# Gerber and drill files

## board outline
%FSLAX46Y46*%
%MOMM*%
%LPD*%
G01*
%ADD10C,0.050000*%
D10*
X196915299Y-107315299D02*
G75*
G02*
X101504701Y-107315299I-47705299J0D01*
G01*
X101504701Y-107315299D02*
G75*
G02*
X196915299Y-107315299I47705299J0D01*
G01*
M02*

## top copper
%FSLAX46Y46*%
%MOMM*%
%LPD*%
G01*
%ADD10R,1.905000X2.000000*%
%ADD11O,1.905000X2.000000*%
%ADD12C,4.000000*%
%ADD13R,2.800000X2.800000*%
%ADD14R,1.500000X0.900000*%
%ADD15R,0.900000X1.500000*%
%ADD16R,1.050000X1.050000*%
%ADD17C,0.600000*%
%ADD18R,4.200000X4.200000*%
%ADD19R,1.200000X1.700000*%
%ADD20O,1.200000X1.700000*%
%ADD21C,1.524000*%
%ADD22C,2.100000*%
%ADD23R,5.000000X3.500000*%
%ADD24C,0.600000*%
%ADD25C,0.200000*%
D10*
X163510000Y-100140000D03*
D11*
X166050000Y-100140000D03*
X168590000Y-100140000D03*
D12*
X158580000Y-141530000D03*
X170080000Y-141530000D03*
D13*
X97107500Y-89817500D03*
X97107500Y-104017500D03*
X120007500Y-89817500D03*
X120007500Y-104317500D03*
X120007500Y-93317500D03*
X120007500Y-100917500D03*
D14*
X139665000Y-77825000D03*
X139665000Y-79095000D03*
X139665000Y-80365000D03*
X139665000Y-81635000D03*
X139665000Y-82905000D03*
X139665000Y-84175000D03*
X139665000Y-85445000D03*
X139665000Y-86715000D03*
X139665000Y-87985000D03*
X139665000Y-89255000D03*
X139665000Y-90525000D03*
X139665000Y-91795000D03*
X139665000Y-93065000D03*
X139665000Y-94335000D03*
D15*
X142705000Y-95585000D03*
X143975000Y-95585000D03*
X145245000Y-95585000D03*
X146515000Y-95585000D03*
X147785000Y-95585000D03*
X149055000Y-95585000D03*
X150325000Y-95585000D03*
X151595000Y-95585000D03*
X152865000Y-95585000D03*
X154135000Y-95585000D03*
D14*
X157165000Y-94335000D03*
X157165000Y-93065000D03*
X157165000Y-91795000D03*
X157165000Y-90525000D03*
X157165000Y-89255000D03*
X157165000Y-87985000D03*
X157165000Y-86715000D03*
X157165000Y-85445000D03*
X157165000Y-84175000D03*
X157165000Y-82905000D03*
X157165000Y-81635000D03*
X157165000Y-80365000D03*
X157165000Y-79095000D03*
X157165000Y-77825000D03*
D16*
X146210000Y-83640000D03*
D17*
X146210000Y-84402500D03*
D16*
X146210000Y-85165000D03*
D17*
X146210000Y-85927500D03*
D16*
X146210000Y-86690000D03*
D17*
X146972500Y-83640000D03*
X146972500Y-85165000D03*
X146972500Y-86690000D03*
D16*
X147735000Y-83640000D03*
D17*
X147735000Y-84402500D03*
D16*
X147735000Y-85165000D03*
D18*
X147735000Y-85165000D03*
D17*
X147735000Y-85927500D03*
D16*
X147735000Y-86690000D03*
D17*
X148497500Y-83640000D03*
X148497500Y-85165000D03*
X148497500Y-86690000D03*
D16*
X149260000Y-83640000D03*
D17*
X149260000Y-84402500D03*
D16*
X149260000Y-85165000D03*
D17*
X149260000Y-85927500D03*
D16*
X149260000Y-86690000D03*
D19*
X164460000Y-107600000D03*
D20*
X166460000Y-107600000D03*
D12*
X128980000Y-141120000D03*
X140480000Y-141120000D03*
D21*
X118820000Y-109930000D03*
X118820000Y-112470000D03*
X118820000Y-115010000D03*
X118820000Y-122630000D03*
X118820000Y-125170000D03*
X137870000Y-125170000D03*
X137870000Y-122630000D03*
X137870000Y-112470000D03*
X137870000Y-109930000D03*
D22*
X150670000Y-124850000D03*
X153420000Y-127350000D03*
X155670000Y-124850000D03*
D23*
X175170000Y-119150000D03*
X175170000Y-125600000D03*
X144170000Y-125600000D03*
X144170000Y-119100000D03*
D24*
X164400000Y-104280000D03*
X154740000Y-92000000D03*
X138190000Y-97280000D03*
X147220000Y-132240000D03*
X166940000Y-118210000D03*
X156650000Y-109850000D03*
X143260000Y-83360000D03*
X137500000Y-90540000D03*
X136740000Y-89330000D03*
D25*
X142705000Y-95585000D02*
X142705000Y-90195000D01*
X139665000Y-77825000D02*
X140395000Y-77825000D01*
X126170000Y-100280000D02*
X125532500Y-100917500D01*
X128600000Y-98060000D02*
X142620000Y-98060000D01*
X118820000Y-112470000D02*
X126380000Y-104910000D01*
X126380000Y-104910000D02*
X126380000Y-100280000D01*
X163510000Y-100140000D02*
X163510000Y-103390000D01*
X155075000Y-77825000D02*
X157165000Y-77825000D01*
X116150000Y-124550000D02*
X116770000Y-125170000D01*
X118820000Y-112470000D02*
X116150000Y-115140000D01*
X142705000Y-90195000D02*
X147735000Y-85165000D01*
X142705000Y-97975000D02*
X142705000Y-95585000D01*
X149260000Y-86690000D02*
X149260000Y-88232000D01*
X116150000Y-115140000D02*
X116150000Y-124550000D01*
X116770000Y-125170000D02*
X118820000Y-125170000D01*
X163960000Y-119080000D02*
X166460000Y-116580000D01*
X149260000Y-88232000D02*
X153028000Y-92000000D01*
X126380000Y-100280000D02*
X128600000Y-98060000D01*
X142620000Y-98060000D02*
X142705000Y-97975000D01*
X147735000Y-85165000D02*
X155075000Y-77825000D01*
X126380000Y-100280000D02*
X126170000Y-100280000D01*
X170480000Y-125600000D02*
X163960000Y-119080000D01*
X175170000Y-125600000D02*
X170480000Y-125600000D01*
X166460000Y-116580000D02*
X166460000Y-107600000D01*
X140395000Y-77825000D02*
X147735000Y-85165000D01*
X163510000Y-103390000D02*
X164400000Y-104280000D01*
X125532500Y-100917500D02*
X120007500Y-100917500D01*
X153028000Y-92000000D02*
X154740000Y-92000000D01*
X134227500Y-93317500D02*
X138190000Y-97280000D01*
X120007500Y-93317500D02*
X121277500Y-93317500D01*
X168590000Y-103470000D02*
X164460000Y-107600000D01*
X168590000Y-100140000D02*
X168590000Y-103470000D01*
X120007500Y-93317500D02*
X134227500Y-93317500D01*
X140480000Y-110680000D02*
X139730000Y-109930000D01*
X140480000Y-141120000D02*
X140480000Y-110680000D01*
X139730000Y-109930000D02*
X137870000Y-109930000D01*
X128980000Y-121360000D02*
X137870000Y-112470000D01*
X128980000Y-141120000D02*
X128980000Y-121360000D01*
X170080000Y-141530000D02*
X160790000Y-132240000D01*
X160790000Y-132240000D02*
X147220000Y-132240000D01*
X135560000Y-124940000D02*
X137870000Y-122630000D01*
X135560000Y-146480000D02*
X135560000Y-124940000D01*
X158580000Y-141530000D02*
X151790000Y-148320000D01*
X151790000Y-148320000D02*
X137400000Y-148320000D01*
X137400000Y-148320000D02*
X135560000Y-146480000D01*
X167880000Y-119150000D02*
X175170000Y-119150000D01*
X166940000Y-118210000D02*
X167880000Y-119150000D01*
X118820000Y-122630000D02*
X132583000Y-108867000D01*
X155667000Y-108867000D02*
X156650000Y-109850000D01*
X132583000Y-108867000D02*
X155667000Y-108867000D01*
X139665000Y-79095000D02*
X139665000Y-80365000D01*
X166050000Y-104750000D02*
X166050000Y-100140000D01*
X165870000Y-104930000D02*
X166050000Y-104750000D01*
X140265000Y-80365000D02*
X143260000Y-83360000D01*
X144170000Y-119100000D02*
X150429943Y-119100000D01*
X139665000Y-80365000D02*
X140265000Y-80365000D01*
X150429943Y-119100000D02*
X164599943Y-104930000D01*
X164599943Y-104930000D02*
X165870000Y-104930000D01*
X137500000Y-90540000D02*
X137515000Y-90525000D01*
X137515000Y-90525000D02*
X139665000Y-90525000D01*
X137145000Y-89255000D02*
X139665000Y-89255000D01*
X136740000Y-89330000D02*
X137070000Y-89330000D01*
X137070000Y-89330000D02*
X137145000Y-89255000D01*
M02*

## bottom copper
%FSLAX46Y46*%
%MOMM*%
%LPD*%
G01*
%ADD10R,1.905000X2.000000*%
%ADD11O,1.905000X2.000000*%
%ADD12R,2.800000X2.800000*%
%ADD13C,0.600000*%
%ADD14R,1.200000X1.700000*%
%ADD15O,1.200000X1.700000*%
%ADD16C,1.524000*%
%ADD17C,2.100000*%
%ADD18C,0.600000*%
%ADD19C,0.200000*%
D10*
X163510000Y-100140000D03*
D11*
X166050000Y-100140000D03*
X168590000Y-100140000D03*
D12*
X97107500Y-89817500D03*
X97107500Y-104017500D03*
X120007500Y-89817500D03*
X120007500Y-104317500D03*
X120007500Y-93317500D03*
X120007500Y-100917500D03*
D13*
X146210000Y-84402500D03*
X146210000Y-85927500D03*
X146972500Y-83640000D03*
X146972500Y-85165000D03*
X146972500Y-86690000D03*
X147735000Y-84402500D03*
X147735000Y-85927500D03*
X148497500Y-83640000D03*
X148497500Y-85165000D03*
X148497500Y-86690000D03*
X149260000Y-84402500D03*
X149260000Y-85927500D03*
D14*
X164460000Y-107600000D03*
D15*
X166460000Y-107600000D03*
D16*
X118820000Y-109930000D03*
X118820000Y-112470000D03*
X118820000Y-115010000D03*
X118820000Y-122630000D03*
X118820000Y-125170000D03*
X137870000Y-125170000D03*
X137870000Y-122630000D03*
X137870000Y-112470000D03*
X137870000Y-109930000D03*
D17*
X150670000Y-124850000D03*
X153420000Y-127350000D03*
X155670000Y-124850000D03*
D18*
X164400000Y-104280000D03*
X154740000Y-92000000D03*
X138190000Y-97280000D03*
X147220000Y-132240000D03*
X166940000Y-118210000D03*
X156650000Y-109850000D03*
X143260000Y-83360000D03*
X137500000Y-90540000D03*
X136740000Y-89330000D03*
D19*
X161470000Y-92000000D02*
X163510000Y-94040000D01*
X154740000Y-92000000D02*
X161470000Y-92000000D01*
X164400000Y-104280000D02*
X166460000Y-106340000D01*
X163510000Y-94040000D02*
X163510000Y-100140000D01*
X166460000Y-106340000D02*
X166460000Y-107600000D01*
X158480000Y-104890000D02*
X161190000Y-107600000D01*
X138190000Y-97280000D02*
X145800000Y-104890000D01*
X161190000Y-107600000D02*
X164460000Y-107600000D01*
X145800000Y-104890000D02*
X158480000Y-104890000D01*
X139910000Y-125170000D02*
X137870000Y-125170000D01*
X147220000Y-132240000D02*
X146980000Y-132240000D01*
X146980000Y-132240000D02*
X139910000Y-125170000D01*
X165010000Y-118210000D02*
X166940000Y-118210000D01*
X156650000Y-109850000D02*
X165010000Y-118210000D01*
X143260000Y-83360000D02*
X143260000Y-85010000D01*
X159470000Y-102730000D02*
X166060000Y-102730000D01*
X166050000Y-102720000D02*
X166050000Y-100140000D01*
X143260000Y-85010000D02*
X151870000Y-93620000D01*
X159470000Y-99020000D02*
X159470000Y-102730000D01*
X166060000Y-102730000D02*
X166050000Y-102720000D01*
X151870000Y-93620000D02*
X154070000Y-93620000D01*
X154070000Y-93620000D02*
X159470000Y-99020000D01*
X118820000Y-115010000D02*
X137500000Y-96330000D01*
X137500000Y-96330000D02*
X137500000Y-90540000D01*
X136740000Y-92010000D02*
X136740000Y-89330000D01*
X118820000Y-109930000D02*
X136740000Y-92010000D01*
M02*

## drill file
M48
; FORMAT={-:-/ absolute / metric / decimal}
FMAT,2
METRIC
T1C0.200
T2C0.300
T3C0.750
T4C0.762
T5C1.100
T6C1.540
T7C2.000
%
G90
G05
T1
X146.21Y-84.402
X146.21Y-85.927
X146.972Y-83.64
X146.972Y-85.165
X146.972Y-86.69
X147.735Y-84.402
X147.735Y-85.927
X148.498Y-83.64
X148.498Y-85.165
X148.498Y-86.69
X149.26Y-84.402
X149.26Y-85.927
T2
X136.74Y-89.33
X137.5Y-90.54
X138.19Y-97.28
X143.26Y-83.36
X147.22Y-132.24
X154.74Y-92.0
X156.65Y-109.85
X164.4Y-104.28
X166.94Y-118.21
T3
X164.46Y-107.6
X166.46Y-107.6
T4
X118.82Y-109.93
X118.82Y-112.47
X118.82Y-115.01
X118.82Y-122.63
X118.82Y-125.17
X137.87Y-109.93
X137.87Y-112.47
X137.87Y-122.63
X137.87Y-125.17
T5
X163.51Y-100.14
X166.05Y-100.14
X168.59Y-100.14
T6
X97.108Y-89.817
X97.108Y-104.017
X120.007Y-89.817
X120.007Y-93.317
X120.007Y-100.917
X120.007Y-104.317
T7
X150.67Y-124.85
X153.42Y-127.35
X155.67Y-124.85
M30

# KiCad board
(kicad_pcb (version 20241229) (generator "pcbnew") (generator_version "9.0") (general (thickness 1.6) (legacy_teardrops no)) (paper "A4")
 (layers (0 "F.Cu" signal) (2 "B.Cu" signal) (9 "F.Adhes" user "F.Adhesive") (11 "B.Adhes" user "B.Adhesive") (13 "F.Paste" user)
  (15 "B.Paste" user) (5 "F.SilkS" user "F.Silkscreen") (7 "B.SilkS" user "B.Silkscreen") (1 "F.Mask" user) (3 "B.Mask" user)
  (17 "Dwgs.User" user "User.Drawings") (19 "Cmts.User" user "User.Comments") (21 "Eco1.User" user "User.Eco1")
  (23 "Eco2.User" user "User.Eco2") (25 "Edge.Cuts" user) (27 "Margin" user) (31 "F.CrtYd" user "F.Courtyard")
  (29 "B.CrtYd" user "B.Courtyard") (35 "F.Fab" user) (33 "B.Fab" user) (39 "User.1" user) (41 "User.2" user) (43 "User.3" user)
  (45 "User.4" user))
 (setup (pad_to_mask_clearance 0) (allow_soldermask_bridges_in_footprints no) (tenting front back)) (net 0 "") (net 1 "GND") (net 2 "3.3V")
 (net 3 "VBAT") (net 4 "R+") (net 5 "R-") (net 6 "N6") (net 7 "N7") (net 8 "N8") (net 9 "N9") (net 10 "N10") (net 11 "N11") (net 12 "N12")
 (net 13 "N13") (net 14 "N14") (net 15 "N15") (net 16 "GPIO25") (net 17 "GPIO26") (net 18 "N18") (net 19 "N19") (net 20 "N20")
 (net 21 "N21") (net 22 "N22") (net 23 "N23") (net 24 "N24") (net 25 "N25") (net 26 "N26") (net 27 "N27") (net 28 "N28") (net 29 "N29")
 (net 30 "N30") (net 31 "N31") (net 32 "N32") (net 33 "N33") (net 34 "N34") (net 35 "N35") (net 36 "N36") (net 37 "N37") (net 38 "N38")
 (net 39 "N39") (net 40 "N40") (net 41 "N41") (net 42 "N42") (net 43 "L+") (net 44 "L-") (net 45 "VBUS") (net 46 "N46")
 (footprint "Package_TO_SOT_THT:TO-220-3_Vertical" (layer "F.Cu") (at 163.51 100.14)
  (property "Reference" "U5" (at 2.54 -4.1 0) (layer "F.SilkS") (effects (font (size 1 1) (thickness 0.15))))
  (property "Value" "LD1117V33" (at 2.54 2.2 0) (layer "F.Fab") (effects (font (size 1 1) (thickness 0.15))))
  (pad "1" thru_hole rect (at 0 0) (size 1.905 2) (drill 1.1) (layers "*.Cu" "*.Mask") (remove_unused_layers no) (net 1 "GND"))
  (pad "2" thru_hole oval (at 2.54 0) (size 1.905 2) (drill 1.1) (layers "*.Cu" "*.Mask") (remove_unused_layers no) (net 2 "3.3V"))
  (pad "3" thru_hole oval (at 5.08 0) (size 1.905 2) (drill 1.1) (layers "*.Cu" "*.Mask") (remove_unused_layers no) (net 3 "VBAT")))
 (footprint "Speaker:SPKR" (layer "F.Cu") (at 165.08 134.03)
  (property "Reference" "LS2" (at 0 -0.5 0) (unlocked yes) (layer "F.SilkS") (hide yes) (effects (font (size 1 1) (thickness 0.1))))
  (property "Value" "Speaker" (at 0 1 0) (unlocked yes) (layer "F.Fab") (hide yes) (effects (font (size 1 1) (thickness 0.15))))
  (pad "1" smd circle (at -6.5 7.5) (size 4 4) (layers "F.Cu" "F.Mask" "F.Paste") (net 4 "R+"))
  (pad "2" smd circle (at 5 7.5) (size 4 4) (layers "F.Cu" "F.Mask" "F.Paste") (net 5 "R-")))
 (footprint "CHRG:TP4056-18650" (layer "F.Cu") (at 95.4075 88.1175)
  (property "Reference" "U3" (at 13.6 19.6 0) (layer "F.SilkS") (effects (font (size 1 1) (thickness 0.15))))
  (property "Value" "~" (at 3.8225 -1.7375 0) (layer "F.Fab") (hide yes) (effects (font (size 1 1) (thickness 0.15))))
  (pad "1" thru_hole rect (at 1.7 1.7) (size 2.8 2.8) (drill 1.54) (layers "*.Cu" "*.Mask") (remove_unused_layers no) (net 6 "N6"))
  (pad "2" thru_hole rect (at 1.7 15.9) (size 2.8 2.8) (drill 1.54) (layers "*.Cu" "*.Mask") (remove_unused_layers no) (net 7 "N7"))
  (pad "3" thru_hole rect (at 24.6 1.7) (size 2.8 2.8) (drill 1.54) (layers "*.Cu" "*.Mask") (remove_unused_layers no) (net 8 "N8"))
  (pad "4" thru_hole rect (at 24.6 16.2) (size 2.8 2.8) (drill 1.54) (layers "*.Cu" "*.Mask") (remove_unused_layers no) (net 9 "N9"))
  (pad "5" thru_hole rect (at 24.6 5.2) (size 2.8 2.8) (drill 1.54) (layers "*.Cu" "*.Mask") (remove_unused_layers no) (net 3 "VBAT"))
  (pad "6" thru_hole rect (at 24.6 12.8) (size 2.8 2.8) (drill 1.54) (layers "*.Cu" "*.Mask") (remove_unused_layers no) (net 1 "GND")))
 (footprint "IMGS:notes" (layer "F.Cu") (at 181.631489 109.410827 -90)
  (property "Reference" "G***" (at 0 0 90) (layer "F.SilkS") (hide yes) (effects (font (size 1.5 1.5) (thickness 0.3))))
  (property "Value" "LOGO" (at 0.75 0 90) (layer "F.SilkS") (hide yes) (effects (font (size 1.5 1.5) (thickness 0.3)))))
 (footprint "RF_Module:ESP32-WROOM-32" (layer "F.Cu") (at 148.415 86.075)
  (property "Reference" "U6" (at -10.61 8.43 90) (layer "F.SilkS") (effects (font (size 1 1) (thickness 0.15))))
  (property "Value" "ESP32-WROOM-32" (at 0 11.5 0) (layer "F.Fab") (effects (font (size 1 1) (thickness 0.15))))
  (pad "1" smd rect (at -8.75 -8.25) (size 1.5 0.9) (layers "F.Cu" "F.Mask" "F.Paste") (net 1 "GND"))
  (pad "2" smd rect (at -8.75 -6.98) (size 1.5 0.9) (layers "F.Cu" "F.Mask" "F.Paste") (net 2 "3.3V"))
  (pad "3" smd rect (at -8.75 -5.71) (size 1.5 0.9) (layers "F.Cu" "F.Mask" "F.Paste") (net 2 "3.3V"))
  (pad "4" smd rect (at -8.75 -4.44) (size 1.5 0.9) (layers "F.Cu" "F.Mask" "F.Paste") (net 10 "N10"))
  (pad "5" smd rect (at -8.75 -3.17) (size 1.5 0.9) (layers "F.Cu" "F.Mask" "F.Paste") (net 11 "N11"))
  (pad "6" smd rect (at -8.75 -1.9) (size 1.5 0.9) (layers "F.Cu" "F.Mask" "F.Paste") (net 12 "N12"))
  (pad "7" smd rect (at -8.75 -0.63) (size 1.5 0.9) (layers "F.Cu" "F.Mask" "F.Paste") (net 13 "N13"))
  (pad "8" smd rect (at -8.75 0.64) (size 1.5 0.9) (layers "F.Cu" "F.Mask" "F.Paste") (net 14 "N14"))
  (pad "9" smd rect (at -8.75 1.91) (size 1.5 0.9) (layers "F.Cu" "F.Mask" "F.Paste") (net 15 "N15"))
  (pad "10" smd rect (at -8.75 3.18) (size 1.5 0.9) (layers "F.Cu" "F.Mask" "F.Paste") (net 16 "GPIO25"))
  (pad "11" smd rect (at -8.75 4.45) (size 1.5 0.9) (layers "F.Cu" "F.Mask" "F.Paste") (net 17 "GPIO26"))
  (pad "12" smd rect (at -8.75 5.72) (size 1.5 0.9) (layers "F.Cu" "F.Mask" "F.Paste") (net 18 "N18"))
  (pad "13" smd rect (at -8.75 6.99) (size 1.5 0.9) (layers "F.Cu" "F.Mask" "F.Paste") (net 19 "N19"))
  (pad "14" smd rect (at -8.75 8.26) (size 1.5 0.9) (layers "F.Cu" "F.Mask" "F.Paste") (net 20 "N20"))
  (pad "15" smd rect (at -5.71 9.51 90) (size 1.5 0.9) (layers "F.Cu" "F.Mask" "F.Paste") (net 1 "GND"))
  (pad "16" smd rect (at -4.44 9.51 90) (size 1.5 0.9) (layers "F.Cu" "F.Mask" "F.Paste") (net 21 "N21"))
  (pad "17" smd rect (at -3.17 9.51 90) (size 1.5 0.9) (layers "F.Cu" "F.Mask" "F.Paste") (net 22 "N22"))
  (pad "18" smd rect (at -1.9 9.51 90) (size 1.5 0.9) (layers "F.Cu" "F.Mask" "F.Paste") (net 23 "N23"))
  (pad "19" smd rect (at -0.63 9.51 90) (size 1.5 0.9) (layers "F.Cu" "F.Mask" "F.Paste") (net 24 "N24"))
  (pad "20" smd rect (at 0.64 9.51 90) (size 1.5 0.9) (layers "F.Cu" "F.Mask" "F.Paste") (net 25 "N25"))
  (pad "21" smd rect (at 1.91 9.51 90) (size 1.5 0.9) (layers "F.Cu" "F.Mask" "F.Paste") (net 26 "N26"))
  (pad "22" smd rect (at 3.18 9.51 90) (size 1.5 0.9) (layers "F.Cu" "F.Mask" "F.Paste") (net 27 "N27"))
  (pad "23" smd rect (at 4.45 9.51 90) (size 1.5 0.9) (layers "F.Cu" "F.Mask" "F.Paste") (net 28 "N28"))
  (pad "24" smd rect (at 5.72 9.51 90) (size 1.5 0.9) (layers "F.Cu" "F.Mask" "F.Paste") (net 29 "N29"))
  (pad "25" smd rect (at 8.75 8.26) (size 1.5 0.9) (layers "F.Cu" "F.Mask" "F.Paste") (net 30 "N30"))
  (pad "26" smd rect (at 8.75 6.99) (size 1.5 0.9) (layers "F.Cu" "F.Mask" "F.Paste") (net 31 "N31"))
  (pad "27" smd rect (at 8.75 5.72) (size 1.5 0.9) (layers "F.Cu" "F.Mask" "F.Paste") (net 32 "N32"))
  (pad "28" smd rect (at 8.75 4.45) (size 1.5 0.9) (layers "F.Cu" "F.Mask" "F.Paste") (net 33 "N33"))
  (pad "29" smd rect (at 8.75 3.18) (size 1.5 0.9) (layers "F.Cu" "F.Mask" "F.Paste") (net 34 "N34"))
  (pad "30" smd rect (at 8.75 1.91) (size 1.5 0.9) (layers "F.Cu" "F.Mask" "F.Paste") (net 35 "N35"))
  (pad "31" smd rect (at 8.75 0.64) (size 1.5 0.9) (layers "F.Cu" "F.Mask" "F.Paste") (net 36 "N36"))
  (pad "32" smd rect (at 8.75 -0.63) (size 1.5 0.9) (layers "F.Cu" "F.Mask" "F.Paste") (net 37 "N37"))
  (pad "33" smd rect (at 8.75 -1.9) (size 1.5 0.9) (layers "F.Cu" "F.Mask" "F.Paste") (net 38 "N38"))
  (pad "34" smd rect (at 8.75 -3.17) (size 1.5 0.9) (layers "F.Cu" "F.Mask" "F.Paste") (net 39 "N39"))
  (pad "35" smd rect (at 8.75 -4.44) (size 1.5 0.9) (layers "F.Cu" "F.Mask" "F.Paste") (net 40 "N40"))
  (pad "36" smd rect (at 8.75 -5.71) (size 1.5 0.9) (layers "F.Cu" "F.Mask" "F.Paste") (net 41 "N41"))
  (pad "37" smd rect (at 8.75 -6.98) (size 1.5 0.9) (layers "F.Cu" "F.Mask" "F.Paste") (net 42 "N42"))
  (pad "38" smd rect (at 8.75 -8.25) (size 1.5 0.9) (layers "F.Cu" "F.Mask" "F.Paste") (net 1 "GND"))
  (pad "39" smd rect (at -2.205 -2.435) (size 1.05 1.05) (layers "F.Cu" "F.Paste") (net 1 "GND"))
  (pad "39" thru_hole circle (at -2.205 -1.6725) (size 0.6 0.6) (drill 0.2) (layers "*.Cu" "F.Mask") (remove_unused_layers no) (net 1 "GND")
   (zone_connect 2))
  (pad "39" smd rect (at -2.205 -0.91) (size 1.05 1.05) (layers "F.Cu" "F.Paste") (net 1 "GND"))
  (pad "39" thru_hole circle (at -2.205 -0.1475) (size 0.6 0.6) (drill 0.2) (layers "*.Cu" "F.Mask") (remove_unused_layers no) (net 1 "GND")
   (zone_connect 2))
  (pad "39" smd rect (at -2.205 0.615) (size 1.05 1.05) (layers "F.Cu" "F.Paste") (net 1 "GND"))
  (pad "39" thru_hole circle (at -1.4425 -2.435) (size 0.6 0.6) (drill 0.2) (layers "*.Cu" "F.Mask") (remove_unused_layers no) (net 1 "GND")
   (zone_connect 2))
  (pad "39" thru_hole circle (at -1.4425 -0.91) (size 0.6 0.6) (drill 0.2) (layers "*.Cu" "F.Mask") (remove_unused_layers no) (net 1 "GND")
   (zone_connect 2))
  (pad "39" thru_hole circle (at -1.4425 0.615) (size 0.6 0.6) (drill 0.2) (layers "*.Cu" "F.Mask") (remove_unused_layers no) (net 1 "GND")
   (zone_connect 2))
  (pad "39" smd rect (at -0.68 -2.435) (size 1.05 1.05) (layers "F.Cu" "F.Paste") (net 1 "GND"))
  (pad "39" thru_hole circle (at -0.68 -1.6725) (size 0.6 0.6) (drill 0.2) (layers "*.Cu" "F.Mask") (remove_unused_layers no) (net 1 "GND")
   (zone_connect 2))
  (pad "39" smd rect (at -0.68 -0.91) (size 1.05 1.05) (layers "F.Cu" "F.Paste") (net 1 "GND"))
  (pad "39" smd rect (at -0.68 -0.91) (size 4.2 4.2) (layers "F.Cu" "F.Mask") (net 1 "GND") (zone_connect 2))
  (pad "39" thru_hole circle (at -0.68 -0.1475) (size 0.6 0.6) (drill 0.2) (layers "*.Cu" "F.Mask") (remove_unused_layers no) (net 1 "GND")
   (zone_connect 2))
  (pad "39" smd rect (at -0.68 0.615) (size 1.05 1.05) (layers "F.Cu" "F.Paste") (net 1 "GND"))
  (pad "39" thru_hole circle (at 0.0825 -2.435) (size 0.6 0.6) (drill 0.2) (layers "*.Cu" "F.Mask") (remove_unused_layers no) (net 1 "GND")
   (zone_connect 2))
  (pad "39" thru_hole circle (at 0.0825 -0.91) (size 0.6 0.6) (drill 0.2) (layers "*.Cu" "F.Mask") (remove_unused_layers no) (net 1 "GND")
   (zone_connect 2))
  (pad "39" thru_hole circle (at 0.0825 0.615) (size 0.6 0.6) (drill 0.2) (layers "*.Cu" "F.Mask") (remove_unused_layers no) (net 1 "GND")
   (zone_connect 2))
  (pad "39" smd rect (at 0.845 -2.435) (size 1.05 1.05) (layers "F.Cu" "F.Paste") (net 1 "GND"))
  (pad "39" thru_hole circle (at 0.845 -1.6725) (size 0.6 0.6) (drill 0.2) (layers "*.Cu" "F.Mask") (remove_unused_layers no) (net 1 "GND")
   (zone_connect 2))
  (pad "39" smd rect (at 0.845 -0.91) (size 1.05 1.05) (layers "F.Cu" "F.Paste") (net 1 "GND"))
  (pad "39" thru_hole circle (at 0.845 -0.1475) (size 0.6 0.6) (drill 0.2) (layers "*.Cu" "F.Mask") (remove_unused_layers no) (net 1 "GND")
   (zone_connect 2))
  (pad "39" smd rect (at 0.845 0.615) (size 1.05 1.05) (layers "F.Cu" "F.Paste") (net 1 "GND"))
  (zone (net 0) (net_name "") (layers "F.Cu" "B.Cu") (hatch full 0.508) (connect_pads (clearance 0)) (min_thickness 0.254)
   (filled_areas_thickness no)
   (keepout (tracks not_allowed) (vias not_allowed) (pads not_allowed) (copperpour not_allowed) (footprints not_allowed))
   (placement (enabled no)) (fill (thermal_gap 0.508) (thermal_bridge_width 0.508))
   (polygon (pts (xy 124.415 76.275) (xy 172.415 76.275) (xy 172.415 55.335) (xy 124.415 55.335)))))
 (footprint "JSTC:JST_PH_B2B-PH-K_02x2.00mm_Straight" (layer "F.Cu") (at 164.46 107.6)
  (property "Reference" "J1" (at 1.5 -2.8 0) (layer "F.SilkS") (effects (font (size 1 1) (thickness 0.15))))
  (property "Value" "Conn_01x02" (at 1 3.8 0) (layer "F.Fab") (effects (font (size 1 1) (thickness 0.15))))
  (pad "1" thru_hole rect (at 0 0) (size 1.2 1.7) (drill 0.75) (layers "*.Cu" "*.Mask") (remove_unused_layers no) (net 3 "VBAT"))
  (pad "2" thru_hole oval (at 2 0) (size 1.2 1.7) (drill 0.75) (layers "*.Cu" "*.Mask") (remove_unused_layers no) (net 1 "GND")))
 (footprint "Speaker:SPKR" (layer "F.Cu") (at 135.48 133.62)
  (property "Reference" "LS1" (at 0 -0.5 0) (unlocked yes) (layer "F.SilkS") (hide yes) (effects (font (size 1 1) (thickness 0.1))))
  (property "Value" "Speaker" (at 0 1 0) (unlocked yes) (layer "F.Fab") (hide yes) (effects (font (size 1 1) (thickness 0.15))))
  (pad "1" smd circle (at -6.5 7.5) (size 4 4) (layers "F.Cu" "F.Mask" "F.Paste") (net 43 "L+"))
  (pad "2" smd circle (at 5 7.5) (size 4 4) (layers "F.Cu" "F.Mask" "F.Paste") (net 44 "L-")))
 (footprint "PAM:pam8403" (layer "F.Cu") (at 128.98 117.55 -90)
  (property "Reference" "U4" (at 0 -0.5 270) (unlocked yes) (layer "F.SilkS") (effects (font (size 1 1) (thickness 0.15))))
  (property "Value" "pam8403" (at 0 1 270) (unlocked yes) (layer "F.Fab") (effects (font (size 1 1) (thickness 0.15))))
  (pad "1" thru_hole circle (at -7.62 10.16 270) (size 1.524 1.524) (drill 0.762) (layers "*.Cu" "*.Mask") (remove_unused_layers no)
   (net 16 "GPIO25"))
  (pad "2" thru_hole circle (at -5.08 10.16 270) (size 1.524 1.524) (drill 0.762) (layers "*.Cu" "*.Mask") (remove_unused_layers no)
   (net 1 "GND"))
  (pad "3" thru_hole circle (at -2.54 10.16 270) (size 1.524 1.524) (drill 0.762) (layers "*.Cu" "*.Mask") (remove_unused_layers no)
   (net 17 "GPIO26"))
  (pad "4" thru_hole circle (at 5.08 10.16 270) (size 1.524 1.524) (drill 0.762) (layers "*.Cu" "*.Mask") (remove_unused_layers no)
   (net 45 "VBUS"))
  (pad "5" thru_hole circle (at 7.62 10.16 270) (size 1.524 1.524) (drill 0.762) (layers "*.Cu" "*.Mask") (remove_unused_layers no)
   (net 1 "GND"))
  (pad "6" thru_hole circle (at 7.62 -8.89 270) (size 1.524 1.524) (drill 0.762) (layers "*.Cu" "*.Mask") (remove_unused_layers no)
   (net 5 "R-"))
  (pad "7" thru_hole circle (at 5.08 -8.89 270) (size 1.524 1.524) (drill 0.762) (layers "*.Cu" "*.Mask") (remove_unused_layers no)
   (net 4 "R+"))
  (pad "8" thru_hole circle (at -5.08 -8.89 270) (size 1.524 1.524) (drill 0.762) (layers "*.Cu" "*.Mask") (remove_unused_layers no)
   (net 43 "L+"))
  (pad "9" thru_hole circle (at -7.62 -8.89 270) (size 1.524 1.524) (drill 0.762) (layers "*.Cu" "*.Mask") (remove_unused_layers no)
   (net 44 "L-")))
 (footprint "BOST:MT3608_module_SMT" (layer "F.Cu") (at 161.17 122.35)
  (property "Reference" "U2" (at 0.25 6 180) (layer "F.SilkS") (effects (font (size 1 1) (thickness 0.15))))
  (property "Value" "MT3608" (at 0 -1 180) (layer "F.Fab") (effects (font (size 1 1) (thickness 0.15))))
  (pad "" thru_hole circle (at -10.5 2.5) (size 2.1 2.1) (drill 2) (layers "*.Cu" "*.Mask" "F.SilkS") (remove_unused_layers no))
  (pad "" thru_hole circle (at -7.75 5) (size 2.1 2.1) (drill 2) (layers "*.Cu" "*.Mask" "F.SilkS") (remove_unused_layers no))
  (pad "" thru_hole circle (at -5.5 2.5) (size 2.1 2.1) (drill 2) (layers "*.Cu" "*.Mask" "F.SilkS") (remove_unused_layers no))
  (pad "1" smd rect (at 14 -3.2 180) (size 5 3.5) (layers "F.Cu" "F.Mask" "F.Paste") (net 45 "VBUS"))
  (pad "2" smd rect (at 14 3.25 180) (size 5 3.5) (layers "F.Cu" "F.Mask" "F.Paste") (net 1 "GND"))
  (pad "3" smd rect (at -17 3.25 180) (size 5 3.5) (layers "F.Cu" "F.Mask" "F.Paste") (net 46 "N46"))
  (pad "4" smd rect (at -17 -3.25 180) (size 5 3.5) (layers "F.Cu" "F.Mask" "F.Paste") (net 2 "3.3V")))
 (gr_circle (center 149.21 107.315299) (end 115.91 73.155299) (stroke (width 0.05) (type default)) (fill no) (layer "Edge.Cuts"))
 (segment (start 142.705 95.585) (end 142.705 90.195) (width 0.2) (layer "F.Cu") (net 1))
 (segment (start 139.665 77.825) (end 140.395 77.825) (width 0.2) (layer "F.Cu") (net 1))
 (segment (start 126.17 100.28) (end 125.5325 100.9175) (width 0.2) (layer "F.Cu") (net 1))
 (segment (start 128.6 98.06) (end 142.62 98.06) (width 0.2) (layer "F.Cu") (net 1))
 (segment (start 118.82 112.47) (end 126.38 104.91) (width 0.2) (layer "F.Cu") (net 1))
 (segment (start 126.38 104.91) (end 126.38 100.28) (width 0.2) (layer "F.Cu") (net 1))
 (segment (start 163.51 100.14) (end 163.51 103.39) (width 0.2) (layer "F.Cu") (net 1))
 (segment (start 155.075 77.825) (end 157.165 77.825) (width 0.2) (layer "F.Cu") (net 1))
 (segment (start 116.15 124.55) (end 116.77 125.17) (width 0.2) (layer "F.Cu") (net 1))
 (segment (start 118.82 112.47) (end 116.15 115.14) (width 0.2) (layer "F.Cu") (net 1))
 (segment (start 142.705 90.195) (end 147.735 85.165) (width 0.2) (layer "F.Cu") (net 1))
 (segment (start 142.705 97.975) (end 142.705 95.585) (width 0.2) (layer "F.Cu") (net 1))
 (segment (start 149.26 86.69) (end 149.26 88.232) (width 0.2) (layer "F.Cu") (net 1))
 (segment (start 116.15 115.14) (end 116.15 124.55) (width 0.2) (layer "F.Cu") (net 1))
 (segment (start 116.77 125.17) (end 118.82 125.17) (width 0.2) (layer "F.Cu") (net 1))
 (segment (start 163.96 119.08) (end 166.46 116.58) (width 0.2) (layer "F.Cu") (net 1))
 (segment (start 149.26 88.232) (end 153.028 92) (width 0.2) (layer "F.Cu") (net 1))
 (segment (start 126.38 100.28) (end 128.6 98.06) (width 0.2) (layer "F.Cu") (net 1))
 (segment (start 142.62 98.06) (end 142.705 97.975) (width 0.2) (layer "F.Cu") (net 1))
 (segment (start 147.735 85.165) (end 155.075 77.825) (width 0.2) (layer "F.Cu") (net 1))
 (segment (start 126.38 100.28) (end 126.17 100.28) (width 0.2) (layer "F.Cu") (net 1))
 (segment (start 170.48 125.6) (end 163.96 119.08) (width 0.2) (layer "F.Cu") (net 1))
 (segment (start 175.17 125.6) (end 170.48 125.6) (width 0.2) (layer "F.Cu") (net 1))
 (segment (start 166.46 116.58) (end 166.46 107.6) (width 0.2) (layer "F.Cu") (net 1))
 (segment (start 140.395 77.825) (end 147.735 85.165) (width 0.2) (layer "F.Cu") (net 1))
 (segment (start 163.51 103.39) (end 164.4 104.28) (width 0.2) (layer "F.Cu") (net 1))
 (segment (start 125.5325 100.9175) (end 120.0075 100.9175) (width 0.2) (layer "F.Cu") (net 1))
 (segment (start 153.028 92) (end 154.74 92) (width 0.2) (layer "F.Cu") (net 1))
 (via (at 164.4 104.28) (size 0.6) (drill 0.3) (layers "F.Cu" "B.Cu") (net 1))
 (via (at 154.74 92) (size 0.6) (drill 0.3) (layers "F.Cu" "B.Cu") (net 1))
 (segment (start 161.47 92) (end 163.51 94.04) (width 0.2) (layer "B.Cu") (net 1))
 (segment (start 154.74 92) (end 161.47 92) (width 0.2) (layer "B.Cu") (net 1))
 (segment (start 164.4 104.28) (end 166.46 106.34) (width 0.2) (layer "B.Cu") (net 1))
 (segment (start 163.51 94.04) (end 163.51 100.14) (width 0.2) (layer "B.Cu") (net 1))
 (segment (start 166.46 106.34) (end 166.46 107.6) (width 0.2) (layer "B.Cu") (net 1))
 (segment (start 134.2275 93.3175) (end 138.19 97.28) (width 0.2) (layer "F.Cu") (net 3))
 (segment (start 120.0075 93.3175) (end 121.2775 93.3175) (width 0.2) (layer "F.Cu") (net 3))
 (segment (start 168.59 103.47) (end 164.46 107.6) (width 0.2) (layer "F.Cu") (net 3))
 (segment (start 168.59 100.14) (end 168.59 103.47) (width 0.2) (layer "F.Cu") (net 3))
 (segment (start 120.0075 93.3175) (end 134.2275 93.3175) (width 0.2) (layer "F.Cu") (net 3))
 (via (at 138.19 97.28) (size 0.6) (drill 0.3) (layers "F.Cu" "B.Cu") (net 3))
 (segment (start 158.48 104.89) (end 161.19 107.6) (width 0.2) (layer "B.Cu") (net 3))
 (segment (start 138.19 97.28) (end 145.8 104.89) (width 0.2) (layer "B.Cu") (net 3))
 (segment (start 161.19 107.6) (end 164.46 107.6) (width 0.2) (layer "B.Cu") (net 3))
 (segment (start 145.8 104.89) (end 158.48 104.89) (width 0.2) (layer "B.Cu") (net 3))
 (segment (start 140.48 110.68) (end 139.73 109.93) (width 0.2) (layer "F.Cu") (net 44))
 (segment (start 140.48 141.12) (end 140.48 110.68) (width 0.2) (layer "F.Cu") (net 44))
 (segment (start 139.73 109.93) (end 137.87 109.93) (width 0.2) (layer "F.Cu") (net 44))
 (segment (start 128.98 121.36) (end 137.87 112.47) (width 0.2) (layer "F.Cu") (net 43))
 (segment (start 128.98 141.12) (end 128.98 121.36) (width 0.2) (layer "F.Cu") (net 43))
 (segment (start 170.08 141.53) (end 160.79 132.24) (width 0.2) (layer "F.Cu") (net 5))
 (segment (start 160.79 132.24) (end 147.22 132.24) (width 0.2) (layer "F.Cu") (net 5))
 (via (at 147.22 132.24) (size 0.6) (drill 0.3) (layers "F.Cu" "B.Cu") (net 5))
 (segment (start 139.91 125.17) (end 137.87 125.17) (width 0.2) (layer "B.Cu") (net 5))
 (segment (start 147.22 132.24) (end 146.98 132.24) (width 0.2) (layer "B.Cu") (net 5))
 (segment (start 146.98 132.24) (end 139.91 125.17) (width 0.2) (layer "B.Cu") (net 5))
 (segment (start 135.56 124.94) (end 137.87 122.63) (width 0.2) (layer "F.Cu") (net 4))
 (segment (start 135.56 146.48) (end 135.56 124.94) (width 0.2) (layer "F.Cu") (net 4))
 (segment (start 158.58 141.53) (end 151.79 148.32) (width 0.2) (layer "F.Cu") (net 4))
 (segment (start 151.79 148.32) (end 137.4 148.32) (width 0.2) (layer "F.Cu") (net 4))
 (segment (start 137.4 148.32) (end 135.56 146.48) (width 0.2) (layer "F.Cu") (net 4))
 (segment (start 167.88 119.15) (end 175.17 119.15) (width 0.2) (layer "F.Cu") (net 45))
 (segment (start 166.94 118.21) (end 167.88 119.15) (width 0.2) (layer "F.Cu") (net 45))
 (segment (start 118.82 122.63) (end 132.583 108.867) (width 0.2) (layer "F.Cu") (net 45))
 (segment (start 155.667 108.867) (end 156.65 109.85) (width 0.2) (layer "F.Cu") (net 45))
 (segment (start 132.583 108.867) (end 155.667 108.867) (width 0.2) (layer "F.Cu") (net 45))
 (via (at 166.94 118.21) (size 0.6) (drill 0.3) (layers "F.Cu" "B.Cu") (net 45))
 (via (at 156.65 109.85) (size 0.6) (drill 0.3) (layers "F.Cu" "B.Cu") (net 45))
 (segment (start 165.01 118.21) (end 166.94 118.21) (width 0.2) (layer "B.Cu") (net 45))
 (segment (start 156.65 109.85) (end 165.01 118.21) (width 0.2) (layer "B.Cu") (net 45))
 (segment (start 139.665 79.095) (end 139.665 80.365) (width 0.2) (layer "F.Cu") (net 2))
 (segment (start 166.05 104.75) (end 166.05 100.14) (width 0.2) (layer "F.Cu") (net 2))
 (segment (start 165.87 104.93) (end 166.05 104.75) (width 0.2) (layer "F.Cu") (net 2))
 (segment (start 140.265 80.365) (end 143.26 83.36) (width 0.2) (layer "F.Cu") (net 2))
 (segment (start 144.17 119.1) (end 150.429943 119.1) (width 0.2) (layer "F.Cu") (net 2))
 (segment (start 139.665 80.365) (end 140.265 80.365) (width 0.2) (layer "F.Cu") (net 2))
 (segment (start 150.429943 119.1) (end 164.599943 104.93) (width 0.2) (layer "F.Cu") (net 2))
 (segment (start 164.599943 104.93) (end 165.87 104.93) (width 0.2) (layer "F.Cu") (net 2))
 (via (at 143.26 83.36) (size 0.6) (drill 0.3) (layers "F.Cu" "B.Cu") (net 2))
 (segment (start 143.26 83.36) (end 143.26 85.01) (width 0.2) (layer "B.Cu") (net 2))
 (segment (start 159.47 102.73) (end 166.06 102.73) (width 0.2) (layer "B.Cu") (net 2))
 (segment (start 166.05 102.72) (end 166.05 100.14) (width 0.2) (layer "B.Cu") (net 2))
 (segment (start 143.26 85.01) (end 151.87 93.62) (width 0.2) (layer "B.Cu") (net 2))
 (segment (start 159.47 99.02) (end 159.47 102.73) (width 0.2) (layer "B.Cu") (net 2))
 (segment (start 166.06 102.73) (end 166.05 102.72) (width 0.2) (layer "B.Cu") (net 2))
 (segment (start 151.87 93.62) (end 154.07 93.62) (width 0.2) (layer "B.Cu") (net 2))
 (segment (start 154.07 93.62) (end 159.47 99.02) (width 0.2) (layer "B.Cu") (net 2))
 (segment (start 137.5 90.54) (end 137.515 90.525) (width 0.2) (layer "F.Cu") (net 17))
 (segment (start 137.515 90.525) (end 139.665 90.525) (width 0.2) (layer "F.Cu") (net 17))
 (via (at 137.5 90.54) (size 0.6) (drill 0.3) (layers "F.Cu" "B.Cu") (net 17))
 (segment (start 118.82 115.01) (end 137.5 96.33) (width 0.2) (layer "B.Cu") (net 17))
 (segment (start 137.5 96.33) (end 137.5 90.54) (width 0.2) (layer "B.Cu") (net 17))
 (segment (start 137.145 89.255) (end 139.665 89.255) (width 0.2) (layer "F.Cu") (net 16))
 (segment (start 136.74 89.33) (end 137.07 89.33) (width 0.2) (layer "F.Cu") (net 16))
 (segment (start 137.07 89.33) (end 137.145 89.255) (width 0.2) (layer "F.Cu") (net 16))
 (via (at 136.74 89.33) (size 0.6) (drill 0.3) (layers "F.Cu" "B.Cu") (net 16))
 (segment (start 136.74 92.01) (end 136.74 89.33) (width 0.2) (layer "B.Cu") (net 16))
 (segment (start 118.82 109.93) (end 136.74 92.01) (width 0.2) (layer "B.Cu") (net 16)))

